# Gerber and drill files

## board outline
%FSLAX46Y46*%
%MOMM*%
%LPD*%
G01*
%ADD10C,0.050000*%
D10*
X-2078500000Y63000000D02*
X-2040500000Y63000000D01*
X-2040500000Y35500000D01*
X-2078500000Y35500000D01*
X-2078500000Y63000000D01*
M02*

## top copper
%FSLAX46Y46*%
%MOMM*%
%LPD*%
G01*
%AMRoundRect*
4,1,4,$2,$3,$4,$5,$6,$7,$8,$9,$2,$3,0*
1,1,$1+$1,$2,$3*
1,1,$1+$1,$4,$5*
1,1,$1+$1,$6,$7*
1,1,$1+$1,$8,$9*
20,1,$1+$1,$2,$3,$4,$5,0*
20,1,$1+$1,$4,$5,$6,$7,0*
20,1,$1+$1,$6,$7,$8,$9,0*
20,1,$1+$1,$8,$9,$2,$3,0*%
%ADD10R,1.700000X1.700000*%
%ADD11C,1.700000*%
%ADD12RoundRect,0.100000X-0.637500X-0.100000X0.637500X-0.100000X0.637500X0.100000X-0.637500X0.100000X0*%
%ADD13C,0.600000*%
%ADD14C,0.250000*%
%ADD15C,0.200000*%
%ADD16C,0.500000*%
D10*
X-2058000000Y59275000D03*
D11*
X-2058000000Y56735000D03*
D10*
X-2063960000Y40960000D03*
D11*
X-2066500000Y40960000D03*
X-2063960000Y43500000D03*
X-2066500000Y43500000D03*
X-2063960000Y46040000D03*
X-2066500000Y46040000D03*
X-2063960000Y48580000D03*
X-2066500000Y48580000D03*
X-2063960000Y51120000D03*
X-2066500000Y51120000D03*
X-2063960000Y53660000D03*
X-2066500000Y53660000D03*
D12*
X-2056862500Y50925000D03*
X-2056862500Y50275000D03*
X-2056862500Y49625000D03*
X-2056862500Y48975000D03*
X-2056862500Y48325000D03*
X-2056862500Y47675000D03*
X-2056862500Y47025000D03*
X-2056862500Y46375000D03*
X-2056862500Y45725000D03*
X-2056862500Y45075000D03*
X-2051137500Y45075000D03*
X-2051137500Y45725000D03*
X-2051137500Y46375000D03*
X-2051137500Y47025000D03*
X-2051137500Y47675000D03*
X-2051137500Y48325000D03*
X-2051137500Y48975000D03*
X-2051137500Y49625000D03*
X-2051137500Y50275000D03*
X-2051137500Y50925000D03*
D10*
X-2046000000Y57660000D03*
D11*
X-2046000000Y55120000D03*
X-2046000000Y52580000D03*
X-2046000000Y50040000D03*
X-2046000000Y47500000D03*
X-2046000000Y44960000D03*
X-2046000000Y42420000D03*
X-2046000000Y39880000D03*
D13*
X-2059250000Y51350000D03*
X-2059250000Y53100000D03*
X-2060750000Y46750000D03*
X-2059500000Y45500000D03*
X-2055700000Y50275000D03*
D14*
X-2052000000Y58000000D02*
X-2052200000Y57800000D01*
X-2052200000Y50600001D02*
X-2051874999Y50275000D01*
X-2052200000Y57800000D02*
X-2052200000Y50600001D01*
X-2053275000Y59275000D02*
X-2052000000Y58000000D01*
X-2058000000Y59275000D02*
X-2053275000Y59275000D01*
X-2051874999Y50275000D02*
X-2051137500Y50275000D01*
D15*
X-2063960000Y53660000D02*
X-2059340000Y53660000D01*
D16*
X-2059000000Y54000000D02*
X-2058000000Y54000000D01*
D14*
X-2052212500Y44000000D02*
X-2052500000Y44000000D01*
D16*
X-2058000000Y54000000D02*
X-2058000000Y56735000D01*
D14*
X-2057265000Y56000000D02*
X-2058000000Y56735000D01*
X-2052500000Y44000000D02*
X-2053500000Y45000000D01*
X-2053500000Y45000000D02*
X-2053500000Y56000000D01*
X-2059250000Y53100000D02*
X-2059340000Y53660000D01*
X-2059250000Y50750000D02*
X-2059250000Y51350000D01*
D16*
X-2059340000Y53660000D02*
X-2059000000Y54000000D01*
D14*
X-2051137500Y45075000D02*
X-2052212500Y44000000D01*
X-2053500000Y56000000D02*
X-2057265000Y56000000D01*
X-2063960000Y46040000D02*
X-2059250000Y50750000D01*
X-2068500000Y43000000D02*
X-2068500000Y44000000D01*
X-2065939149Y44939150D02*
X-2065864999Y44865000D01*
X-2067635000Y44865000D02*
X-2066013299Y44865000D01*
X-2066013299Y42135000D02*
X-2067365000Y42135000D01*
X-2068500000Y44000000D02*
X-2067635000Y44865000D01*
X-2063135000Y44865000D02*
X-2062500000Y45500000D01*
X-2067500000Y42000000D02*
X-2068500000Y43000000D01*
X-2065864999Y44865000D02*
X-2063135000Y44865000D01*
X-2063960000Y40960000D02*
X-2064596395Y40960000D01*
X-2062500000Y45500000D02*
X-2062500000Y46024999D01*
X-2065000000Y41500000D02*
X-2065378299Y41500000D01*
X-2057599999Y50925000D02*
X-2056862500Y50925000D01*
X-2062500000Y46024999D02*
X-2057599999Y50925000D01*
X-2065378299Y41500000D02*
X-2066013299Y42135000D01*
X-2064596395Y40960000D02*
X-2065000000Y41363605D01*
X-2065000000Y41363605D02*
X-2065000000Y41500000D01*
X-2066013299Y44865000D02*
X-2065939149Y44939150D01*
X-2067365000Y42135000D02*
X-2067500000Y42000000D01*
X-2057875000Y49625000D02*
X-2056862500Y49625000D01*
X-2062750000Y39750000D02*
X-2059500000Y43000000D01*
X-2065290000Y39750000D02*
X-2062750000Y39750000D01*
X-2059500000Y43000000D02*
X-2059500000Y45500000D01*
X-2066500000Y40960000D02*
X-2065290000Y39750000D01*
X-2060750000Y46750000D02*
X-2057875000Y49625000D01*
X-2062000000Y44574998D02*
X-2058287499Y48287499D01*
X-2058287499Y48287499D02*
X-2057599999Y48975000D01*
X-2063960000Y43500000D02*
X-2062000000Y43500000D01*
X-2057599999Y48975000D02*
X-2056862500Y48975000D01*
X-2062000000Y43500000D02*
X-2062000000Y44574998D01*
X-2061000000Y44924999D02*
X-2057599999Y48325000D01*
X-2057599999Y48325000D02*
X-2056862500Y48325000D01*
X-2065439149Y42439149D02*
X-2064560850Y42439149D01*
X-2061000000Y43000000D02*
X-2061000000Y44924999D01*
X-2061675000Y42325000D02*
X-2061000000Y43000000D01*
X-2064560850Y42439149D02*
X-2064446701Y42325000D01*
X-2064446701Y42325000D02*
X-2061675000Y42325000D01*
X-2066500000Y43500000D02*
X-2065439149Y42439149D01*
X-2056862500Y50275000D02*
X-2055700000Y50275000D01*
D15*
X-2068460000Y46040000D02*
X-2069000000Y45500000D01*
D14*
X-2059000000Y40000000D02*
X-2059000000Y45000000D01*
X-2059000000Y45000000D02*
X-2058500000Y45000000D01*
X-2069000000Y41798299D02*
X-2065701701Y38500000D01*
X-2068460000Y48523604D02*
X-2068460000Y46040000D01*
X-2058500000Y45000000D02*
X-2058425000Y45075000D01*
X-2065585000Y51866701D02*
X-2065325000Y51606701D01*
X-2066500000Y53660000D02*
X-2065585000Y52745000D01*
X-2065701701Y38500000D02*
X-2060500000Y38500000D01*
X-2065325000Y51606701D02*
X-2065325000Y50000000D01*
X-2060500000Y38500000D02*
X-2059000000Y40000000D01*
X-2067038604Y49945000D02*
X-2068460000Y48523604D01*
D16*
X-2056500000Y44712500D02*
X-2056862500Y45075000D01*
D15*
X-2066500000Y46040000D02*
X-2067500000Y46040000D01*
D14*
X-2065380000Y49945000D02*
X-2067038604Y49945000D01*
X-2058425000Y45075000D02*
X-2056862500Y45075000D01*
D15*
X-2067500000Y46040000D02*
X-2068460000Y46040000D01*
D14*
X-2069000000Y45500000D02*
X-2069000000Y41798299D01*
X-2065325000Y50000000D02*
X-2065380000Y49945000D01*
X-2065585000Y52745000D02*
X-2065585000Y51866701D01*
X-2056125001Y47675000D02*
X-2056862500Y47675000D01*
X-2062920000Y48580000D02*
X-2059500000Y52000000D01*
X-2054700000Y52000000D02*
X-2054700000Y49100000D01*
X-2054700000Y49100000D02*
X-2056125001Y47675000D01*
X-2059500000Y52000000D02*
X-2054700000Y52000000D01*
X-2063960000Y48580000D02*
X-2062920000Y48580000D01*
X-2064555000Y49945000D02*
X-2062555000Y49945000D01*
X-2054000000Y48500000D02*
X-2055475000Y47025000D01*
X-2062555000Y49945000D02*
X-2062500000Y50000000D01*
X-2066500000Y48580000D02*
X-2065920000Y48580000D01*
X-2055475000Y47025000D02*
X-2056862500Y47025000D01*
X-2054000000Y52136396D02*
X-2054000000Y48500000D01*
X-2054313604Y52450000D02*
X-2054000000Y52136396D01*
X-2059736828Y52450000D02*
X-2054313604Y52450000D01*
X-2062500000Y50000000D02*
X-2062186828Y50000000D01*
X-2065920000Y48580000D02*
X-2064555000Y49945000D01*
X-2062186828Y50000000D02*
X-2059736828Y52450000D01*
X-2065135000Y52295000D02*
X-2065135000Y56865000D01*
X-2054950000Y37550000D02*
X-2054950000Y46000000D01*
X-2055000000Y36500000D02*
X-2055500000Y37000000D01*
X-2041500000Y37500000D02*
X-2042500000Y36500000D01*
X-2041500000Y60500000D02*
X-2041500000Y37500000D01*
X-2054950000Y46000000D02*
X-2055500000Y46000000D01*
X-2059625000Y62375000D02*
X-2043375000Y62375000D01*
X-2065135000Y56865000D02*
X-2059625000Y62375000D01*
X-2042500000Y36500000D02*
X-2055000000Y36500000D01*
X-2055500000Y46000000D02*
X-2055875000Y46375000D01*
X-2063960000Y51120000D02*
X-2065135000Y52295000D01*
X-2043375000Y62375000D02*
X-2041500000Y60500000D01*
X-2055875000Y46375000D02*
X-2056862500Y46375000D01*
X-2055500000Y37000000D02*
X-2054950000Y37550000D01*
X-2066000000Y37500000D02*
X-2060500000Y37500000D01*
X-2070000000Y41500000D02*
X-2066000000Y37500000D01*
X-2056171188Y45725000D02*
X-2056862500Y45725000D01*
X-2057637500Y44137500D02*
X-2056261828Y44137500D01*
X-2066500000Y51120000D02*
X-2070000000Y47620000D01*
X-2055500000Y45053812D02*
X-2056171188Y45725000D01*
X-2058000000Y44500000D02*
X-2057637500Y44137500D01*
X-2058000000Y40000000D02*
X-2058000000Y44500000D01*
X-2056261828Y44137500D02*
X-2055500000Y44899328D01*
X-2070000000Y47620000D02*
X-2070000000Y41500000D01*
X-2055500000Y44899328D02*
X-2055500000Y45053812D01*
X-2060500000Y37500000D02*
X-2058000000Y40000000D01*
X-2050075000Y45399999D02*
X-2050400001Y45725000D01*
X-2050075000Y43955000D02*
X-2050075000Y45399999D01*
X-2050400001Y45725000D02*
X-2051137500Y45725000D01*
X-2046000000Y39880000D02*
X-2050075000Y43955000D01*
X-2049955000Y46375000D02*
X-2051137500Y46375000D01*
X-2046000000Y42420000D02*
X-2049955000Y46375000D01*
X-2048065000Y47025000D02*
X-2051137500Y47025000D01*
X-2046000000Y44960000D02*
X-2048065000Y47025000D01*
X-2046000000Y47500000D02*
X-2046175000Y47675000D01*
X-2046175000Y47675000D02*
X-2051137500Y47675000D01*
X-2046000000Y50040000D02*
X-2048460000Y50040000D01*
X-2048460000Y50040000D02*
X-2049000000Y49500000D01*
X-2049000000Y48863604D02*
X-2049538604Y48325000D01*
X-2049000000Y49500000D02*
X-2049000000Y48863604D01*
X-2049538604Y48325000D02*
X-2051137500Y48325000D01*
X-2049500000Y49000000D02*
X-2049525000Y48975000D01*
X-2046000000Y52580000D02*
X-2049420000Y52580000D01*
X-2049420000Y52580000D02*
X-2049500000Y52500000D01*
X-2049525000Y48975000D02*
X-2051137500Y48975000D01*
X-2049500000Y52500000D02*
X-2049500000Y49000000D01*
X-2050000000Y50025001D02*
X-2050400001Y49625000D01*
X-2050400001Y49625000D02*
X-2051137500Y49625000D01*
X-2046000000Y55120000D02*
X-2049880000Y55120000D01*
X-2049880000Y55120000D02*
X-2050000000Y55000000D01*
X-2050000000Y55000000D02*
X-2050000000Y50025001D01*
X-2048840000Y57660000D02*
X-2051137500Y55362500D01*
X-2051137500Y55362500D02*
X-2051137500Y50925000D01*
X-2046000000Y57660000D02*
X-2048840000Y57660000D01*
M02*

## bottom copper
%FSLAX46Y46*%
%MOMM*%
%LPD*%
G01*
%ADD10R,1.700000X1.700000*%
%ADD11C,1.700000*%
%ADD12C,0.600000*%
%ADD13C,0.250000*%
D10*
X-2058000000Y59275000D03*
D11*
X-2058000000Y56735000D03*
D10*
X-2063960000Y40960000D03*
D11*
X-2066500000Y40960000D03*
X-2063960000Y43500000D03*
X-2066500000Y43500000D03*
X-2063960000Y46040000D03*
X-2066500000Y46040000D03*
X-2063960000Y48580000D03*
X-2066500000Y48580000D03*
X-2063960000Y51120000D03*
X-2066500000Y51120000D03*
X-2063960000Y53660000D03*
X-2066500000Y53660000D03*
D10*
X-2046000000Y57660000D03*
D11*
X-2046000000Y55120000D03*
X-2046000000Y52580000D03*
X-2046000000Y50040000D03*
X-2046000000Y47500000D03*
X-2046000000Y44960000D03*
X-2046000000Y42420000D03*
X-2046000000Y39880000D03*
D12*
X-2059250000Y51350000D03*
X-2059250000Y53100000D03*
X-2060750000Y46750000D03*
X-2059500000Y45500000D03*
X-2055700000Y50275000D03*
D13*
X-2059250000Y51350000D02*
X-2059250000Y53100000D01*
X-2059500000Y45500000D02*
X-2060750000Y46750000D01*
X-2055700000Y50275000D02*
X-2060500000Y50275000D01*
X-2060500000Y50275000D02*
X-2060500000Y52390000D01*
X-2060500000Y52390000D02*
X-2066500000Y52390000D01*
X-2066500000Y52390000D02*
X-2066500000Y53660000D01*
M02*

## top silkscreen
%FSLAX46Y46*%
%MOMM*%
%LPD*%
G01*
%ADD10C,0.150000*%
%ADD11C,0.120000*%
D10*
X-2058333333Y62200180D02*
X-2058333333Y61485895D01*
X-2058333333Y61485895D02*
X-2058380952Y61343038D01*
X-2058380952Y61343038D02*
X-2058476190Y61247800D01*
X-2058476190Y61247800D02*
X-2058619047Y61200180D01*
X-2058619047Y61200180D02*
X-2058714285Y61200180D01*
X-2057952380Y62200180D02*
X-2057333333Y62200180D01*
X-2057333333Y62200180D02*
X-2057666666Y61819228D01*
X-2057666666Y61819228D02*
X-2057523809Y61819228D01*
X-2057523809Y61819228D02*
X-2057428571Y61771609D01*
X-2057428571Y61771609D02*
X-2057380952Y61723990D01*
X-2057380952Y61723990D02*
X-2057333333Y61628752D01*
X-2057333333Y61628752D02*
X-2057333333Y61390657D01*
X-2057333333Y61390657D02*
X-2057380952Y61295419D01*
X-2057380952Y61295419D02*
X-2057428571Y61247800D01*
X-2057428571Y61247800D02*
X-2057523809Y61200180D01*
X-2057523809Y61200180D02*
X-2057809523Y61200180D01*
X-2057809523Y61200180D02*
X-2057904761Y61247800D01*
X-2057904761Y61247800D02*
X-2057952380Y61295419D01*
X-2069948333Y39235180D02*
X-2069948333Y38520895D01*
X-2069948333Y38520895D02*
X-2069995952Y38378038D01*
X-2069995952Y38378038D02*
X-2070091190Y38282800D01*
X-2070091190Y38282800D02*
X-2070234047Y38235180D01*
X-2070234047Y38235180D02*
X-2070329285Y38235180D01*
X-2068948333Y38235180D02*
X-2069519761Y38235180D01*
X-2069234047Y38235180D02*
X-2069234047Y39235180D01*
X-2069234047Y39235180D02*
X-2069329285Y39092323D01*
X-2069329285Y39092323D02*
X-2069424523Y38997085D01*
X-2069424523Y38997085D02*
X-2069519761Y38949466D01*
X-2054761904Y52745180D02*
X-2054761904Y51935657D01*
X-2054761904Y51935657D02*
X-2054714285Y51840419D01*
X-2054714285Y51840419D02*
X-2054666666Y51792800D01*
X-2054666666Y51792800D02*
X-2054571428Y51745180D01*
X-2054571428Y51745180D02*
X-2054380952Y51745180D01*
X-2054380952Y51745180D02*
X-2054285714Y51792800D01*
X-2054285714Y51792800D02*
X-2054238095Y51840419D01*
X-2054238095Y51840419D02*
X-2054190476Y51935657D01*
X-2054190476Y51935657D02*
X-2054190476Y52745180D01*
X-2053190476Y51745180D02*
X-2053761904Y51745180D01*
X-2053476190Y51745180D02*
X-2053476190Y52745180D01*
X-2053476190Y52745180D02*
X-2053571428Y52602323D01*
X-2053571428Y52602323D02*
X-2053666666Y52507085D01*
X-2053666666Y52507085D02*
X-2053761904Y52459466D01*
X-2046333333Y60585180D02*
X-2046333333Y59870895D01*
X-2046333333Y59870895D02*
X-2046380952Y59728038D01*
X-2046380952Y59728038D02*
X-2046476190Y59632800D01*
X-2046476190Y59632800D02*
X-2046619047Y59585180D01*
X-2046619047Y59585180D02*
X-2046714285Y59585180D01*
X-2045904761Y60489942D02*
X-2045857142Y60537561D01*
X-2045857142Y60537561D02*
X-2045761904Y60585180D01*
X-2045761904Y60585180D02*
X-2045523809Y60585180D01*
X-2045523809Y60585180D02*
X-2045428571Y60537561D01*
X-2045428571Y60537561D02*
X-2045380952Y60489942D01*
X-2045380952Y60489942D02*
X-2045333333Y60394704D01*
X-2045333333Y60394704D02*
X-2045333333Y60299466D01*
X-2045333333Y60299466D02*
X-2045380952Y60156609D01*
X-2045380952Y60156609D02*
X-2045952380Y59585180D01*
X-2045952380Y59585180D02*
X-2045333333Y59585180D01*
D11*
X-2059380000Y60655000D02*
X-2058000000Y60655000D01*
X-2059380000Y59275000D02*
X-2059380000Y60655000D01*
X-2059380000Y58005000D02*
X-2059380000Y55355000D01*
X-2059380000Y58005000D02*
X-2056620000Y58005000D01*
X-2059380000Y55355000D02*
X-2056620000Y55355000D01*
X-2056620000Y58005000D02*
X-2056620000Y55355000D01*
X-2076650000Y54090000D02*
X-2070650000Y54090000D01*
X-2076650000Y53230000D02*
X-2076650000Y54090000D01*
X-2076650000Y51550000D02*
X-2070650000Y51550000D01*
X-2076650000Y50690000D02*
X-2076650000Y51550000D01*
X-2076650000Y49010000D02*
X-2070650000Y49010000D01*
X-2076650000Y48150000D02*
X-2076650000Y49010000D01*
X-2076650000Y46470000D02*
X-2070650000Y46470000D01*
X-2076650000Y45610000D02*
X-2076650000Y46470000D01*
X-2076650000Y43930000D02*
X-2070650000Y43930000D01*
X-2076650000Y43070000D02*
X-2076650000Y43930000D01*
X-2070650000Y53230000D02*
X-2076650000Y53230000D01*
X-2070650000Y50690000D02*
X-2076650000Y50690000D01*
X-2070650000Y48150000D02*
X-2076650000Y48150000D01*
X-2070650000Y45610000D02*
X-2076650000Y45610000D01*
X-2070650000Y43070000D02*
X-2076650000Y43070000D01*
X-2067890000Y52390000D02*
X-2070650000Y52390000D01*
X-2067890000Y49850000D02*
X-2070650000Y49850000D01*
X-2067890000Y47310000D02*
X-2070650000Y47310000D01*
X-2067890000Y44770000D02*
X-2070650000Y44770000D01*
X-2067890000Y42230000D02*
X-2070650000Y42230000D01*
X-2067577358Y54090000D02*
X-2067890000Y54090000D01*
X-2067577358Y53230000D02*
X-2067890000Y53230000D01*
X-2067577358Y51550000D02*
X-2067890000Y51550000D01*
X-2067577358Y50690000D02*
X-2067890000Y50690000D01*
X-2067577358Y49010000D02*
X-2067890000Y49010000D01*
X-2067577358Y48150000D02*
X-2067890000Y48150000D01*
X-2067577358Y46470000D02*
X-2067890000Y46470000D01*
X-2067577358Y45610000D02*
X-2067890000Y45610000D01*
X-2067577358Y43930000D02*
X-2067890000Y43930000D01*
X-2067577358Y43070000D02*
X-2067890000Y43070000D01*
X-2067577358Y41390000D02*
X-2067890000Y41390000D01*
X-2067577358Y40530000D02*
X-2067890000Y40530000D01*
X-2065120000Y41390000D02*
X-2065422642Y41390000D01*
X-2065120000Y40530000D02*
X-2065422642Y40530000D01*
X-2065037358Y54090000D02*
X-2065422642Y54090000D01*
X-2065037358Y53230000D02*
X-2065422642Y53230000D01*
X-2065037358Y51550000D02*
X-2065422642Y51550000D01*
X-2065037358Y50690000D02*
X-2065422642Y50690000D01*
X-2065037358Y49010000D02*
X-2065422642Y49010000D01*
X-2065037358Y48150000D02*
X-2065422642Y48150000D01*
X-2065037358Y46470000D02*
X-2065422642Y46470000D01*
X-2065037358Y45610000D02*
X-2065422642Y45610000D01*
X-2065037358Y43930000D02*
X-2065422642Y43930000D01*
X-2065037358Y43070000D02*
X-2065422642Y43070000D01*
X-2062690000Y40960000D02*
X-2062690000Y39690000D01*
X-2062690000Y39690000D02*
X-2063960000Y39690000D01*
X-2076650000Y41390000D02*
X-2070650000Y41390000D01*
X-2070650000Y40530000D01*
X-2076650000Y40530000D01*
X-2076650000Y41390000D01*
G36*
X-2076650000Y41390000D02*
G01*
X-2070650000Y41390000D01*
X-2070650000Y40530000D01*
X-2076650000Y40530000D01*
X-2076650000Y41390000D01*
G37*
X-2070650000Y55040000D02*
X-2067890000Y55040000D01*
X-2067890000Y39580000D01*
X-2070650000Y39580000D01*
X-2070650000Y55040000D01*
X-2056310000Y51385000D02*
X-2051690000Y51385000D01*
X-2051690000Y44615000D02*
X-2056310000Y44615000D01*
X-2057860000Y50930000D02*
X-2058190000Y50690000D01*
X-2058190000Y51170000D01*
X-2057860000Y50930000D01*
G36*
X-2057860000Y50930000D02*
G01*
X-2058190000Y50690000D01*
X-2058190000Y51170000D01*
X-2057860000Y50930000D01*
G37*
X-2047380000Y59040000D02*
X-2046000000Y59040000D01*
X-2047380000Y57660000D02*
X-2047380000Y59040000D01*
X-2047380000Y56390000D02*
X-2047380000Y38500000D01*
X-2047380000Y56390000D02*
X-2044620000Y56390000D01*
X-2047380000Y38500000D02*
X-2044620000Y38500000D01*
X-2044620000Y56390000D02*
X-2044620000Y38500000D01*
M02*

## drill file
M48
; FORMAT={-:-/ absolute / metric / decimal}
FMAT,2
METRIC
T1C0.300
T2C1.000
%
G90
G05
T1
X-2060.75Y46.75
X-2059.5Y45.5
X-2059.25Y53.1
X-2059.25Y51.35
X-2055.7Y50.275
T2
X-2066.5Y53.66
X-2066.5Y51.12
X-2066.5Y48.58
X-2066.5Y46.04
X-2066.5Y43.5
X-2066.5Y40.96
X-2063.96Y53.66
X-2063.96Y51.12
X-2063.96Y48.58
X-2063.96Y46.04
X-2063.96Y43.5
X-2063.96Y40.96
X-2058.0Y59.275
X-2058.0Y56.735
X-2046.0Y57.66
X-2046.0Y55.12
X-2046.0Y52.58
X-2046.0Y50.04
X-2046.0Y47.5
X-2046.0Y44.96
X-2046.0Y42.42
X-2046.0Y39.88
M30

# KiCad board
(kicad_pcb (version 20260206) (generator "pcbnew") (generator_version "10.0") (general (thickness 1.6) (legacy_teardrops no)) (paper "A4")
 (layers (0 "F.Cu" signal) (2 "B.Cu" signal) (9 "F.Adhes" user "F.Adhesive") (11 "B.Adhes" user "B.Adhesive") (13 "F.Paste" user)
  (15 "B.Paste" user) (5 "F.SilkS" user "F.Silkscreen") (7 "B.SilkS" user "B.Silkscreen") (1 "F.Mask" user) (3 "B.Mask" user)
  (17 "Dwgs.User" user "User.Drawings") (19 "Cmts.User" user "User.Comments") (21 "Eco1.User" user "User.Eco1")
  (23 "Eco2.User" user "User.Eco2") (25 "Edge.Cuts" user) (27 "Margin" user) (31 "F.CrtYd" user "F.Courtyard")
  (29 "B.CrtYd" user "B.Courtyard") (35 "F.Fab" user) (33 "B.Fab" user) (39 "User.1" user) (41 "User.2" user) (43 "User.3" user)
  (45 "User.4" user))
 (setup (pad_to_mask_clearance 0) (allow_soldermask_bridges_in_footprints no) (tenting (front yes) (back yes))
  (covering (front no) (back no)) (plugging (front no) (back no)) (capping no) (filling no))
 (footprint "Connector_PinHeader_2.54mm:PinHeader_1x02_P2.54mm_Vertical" (layer "F.Cu") (at -2058 -59.275)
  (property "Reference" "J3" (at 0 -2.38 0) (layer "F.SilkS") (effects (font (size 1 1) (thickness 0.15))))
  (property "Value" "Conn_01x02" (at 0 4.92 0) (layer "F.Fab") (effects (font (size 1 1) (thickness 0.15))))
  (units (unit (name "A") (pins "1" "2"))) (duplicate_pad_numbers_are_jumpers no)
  (fp_line (start -1.38 -1.38) (end 0 -1.38) (stroke (width 0.12) (type solid)) (layer "F.SilkS"))
  (fp_line (start -1.38 0) (end -1.38 -1.38) (stroke (width 0.12) (type solid)) (layer "F.SilkS"))
  (fp_line (start -1.38 1.27) (end -1.38 3.92) (stroke (width 0.12) (type solid)) (layer "F.SilkS"))
  (fp_line (start -1.38 1.27) (end 1.38 1.27) (stroke (width 0.12) (type solid)) (layer "F.SilkS"))
  (fp_line (start -1.38 3.92) (end 1.38 3.92) (stroke (width 0.12) (type solid)) (layer "F.SilkS"))
  (fp_line (start 1.38 1.27) (end 1.38 3.92) (stroke (width 0.12) (type solid)) (layer "F.SilkS"))
  (pad "1" thru_hole rect (at 0 0) (size 1.7 1.7) (drill 1) (layers "*.Cu" "*.Mask") (remove_unused_layers no) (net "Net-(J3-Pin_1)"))
  (pad "2" thru_hole circle (at 0 2.54) (size 1.7 1.7) (drill 1) (layers "*.Cu" "*.Mask") (remove_unused_layers no) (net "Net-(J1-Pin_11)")))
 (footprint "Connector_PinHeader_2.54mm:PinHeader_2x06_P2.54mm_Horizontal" (layer "F.Cu") (at -2063.96 -40.96 180)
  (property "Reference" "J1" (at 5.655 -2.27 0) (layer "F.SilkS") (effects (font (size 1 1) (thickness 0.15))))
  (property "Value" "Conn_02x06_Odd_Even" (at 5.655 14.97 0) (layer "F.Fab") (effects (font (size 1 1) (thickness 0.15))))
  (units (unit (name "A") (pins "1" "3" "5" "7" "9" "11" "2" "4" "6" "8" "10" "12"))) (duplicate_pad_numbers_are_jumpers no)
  (fp_line (start 12.69 13.13) (end 6.69 13.13) (stroke (width 0.12) (type solid)) (layer "F.SilkS"))
  (fp_line (start 12.69 12.27) (end 12.69 13.13) (stroke (width 0.12) (type solid)) (layer "F.SilkS"))
  (fp_line (start 12.69 10.59) (end 6.69 10.59) (stroke (width 0.12) (type solid)) (layer "F.SilkS"))
  (fp_line (start 12.69 9.73) (end 12.69 10.59) (stroke (width 0.12) (type solid)) (layer "F.SilkS"))
  (fp_line (start 12.69 8.05) (end 6.69 8.05) (stroke (width 0.12) (type solid)) (layer "F.SilkS"))
  (fp_line (start 12.69 7.19) (end 12.69 8.05) (stroke (width 0.12) (type solid)) (layer "F.SilkS"))
  (fp_line (start 12.69 5.51) (end 6.69 5.51) (stroke (width 0.12) (type solid)) (layer "F.SilkS"))
  (fp_line (start 12.69 4.65) (end 12.69 5.51) (stroke (width 0.12) (type solid)) (layer "F.SilkS"))
  (fp_line (start 12.69 2.97) (end 6.69 2.97) (stroke (width 0.12) (type solid)) (layer "F.SilkS"))
  (fp_line (start 12.69 2.11) (end 12.69 2.97) (stroke (width 0.12) (type solid)) (layer "F.SilkS"))
  (fp_line (start 6.69 12.27) (end 12.69 12.27) (stroke (width 0.12) (type solid)) (layer "F.SilkS"))
  (fp_line (start 6.69 9.73) (end 12.69 9.73) (stroke (width 0.12) (type solid)) (layer "F.SilkS"))
  (fp_line (start 6.69 7.19) (end 12.69 7.19) (stroke (width 0.12) (type solid)) (layer "F.SilkS"))
  (fp_line (start 6.69 4.65) (end 12.69 4.65) (stroke (width 0.12) (type solid)) (layer "F.SilkS"))
  (fp_line (start 6.69 2.11) (end 12.69 2.11) (stroke (width 0.12) (type solid)) (layer "F.SilkS"))
  (fp_line (start 3.93 11.43) (end 6.69 11.43) (stroke (width 0.12) (type solid)) (layer "F.SilkS"))
  (fp_line (start 3.93 8.89) (end 6.69 8.89) (stroke (width 0.12) (type solid)) (layer "F.SilkS"))
  (fp_line (start 3.93 6.35) (end 6.69 6.35) (stroke (width 0.12) (type solid)) (layer "F.SilkS"))
  (fp_line (start 3.93 3.81) (end 6.69 3.81) (stroke (width 0.12) (type solid)) (layer "F.SilkS"))
  (fp_line (start 3.93 1.27) (end 6.69 1.27) (stroke (width 0.12) (type solid)) (layer "F.SilkS"))
  (fp_line (start 3.617358 13.13) (end 3.93 13.13) (stroke (width 0.12) (type solid)) (layer "F.SilkS"))
  (fp_line (start 3.617358 12.27) (end 3.93 12.27) (stroke (width 0.12) (type solid)) (layer "F.SilkS"))
  (fp_line (start 3.617358 10.59) (end 3.93 10.59) (stroke (width 0.12) (type solid)) (layer "F.SilkS"))
  (fp_line (start 3.617358 9.73) (end 3.93 9.73) (stroke (width 0.12) (type solid)) (layer "F.SilkS"))
  (fp_line (start 3.617358 8.05) (end 3.93 8.05) (stroke (width 0.12) (type solid)) (layer "F.SilkS"))
  (fp_line (start 3.617358 7.19) (end 3.93 7.19) (stroke (width 0.12) (type solid)) (layer "F.SilkS"))
  (fp_line (start 3.617358 5.51) (end 3.93 5.51) (stroke (width 0.12) (type solid)) (layer "F.SilkS"))
  (fp_line (start 3.617358 4.65) (end 3.93 4.65) (stroke (width 0.12) (type solid)) (layer "F.SilkS"))
  (fp_line (start 3.617358 2.97) (end 3.93 2.97) (stroke (width 0.12) (type solid)) (layer "F.SilkS"))
  (fp_line (start 3.617358 2.11) (end 3.93 2.11) (stroke (width 0.12) (type solid)) (layer "F.SilkS"))
  (fp_line (start 3.617358 0.43) (end 3.93 0.43) (stroke (width 0.12) (type solid)) (layer "F.SilkS"))
  (fp_line (start 3.617358 -0.43) (end 3.93 -0.43) (stroke (width 0.12) (type solid)) (layer "F.SilkS"))
  (fp_line (start 1.16 0.43) (end 1.462642 0.43) (stroke (width 0.12) (type solid)) (layer "F.SilkS"))
  (fp_line (start 1.16 -0.43) (end 1.462642 -0.43) (stroke (width 0.12) (type solid)) (layer "F.SilkS"))
  (fp_line (start 1.077358 13.13) (end 1.462642 13.13) (stroke (width 0.12) (type solid)) (layer "F.SilkS"))
  (fp_line (start 1.077358 12.27) (end 1.462642 12.27) (stroke (width 0.12) (type solid)) (layer "F.SilkS"))
  (fp_line (start 1.077358 10.59) (end 1.462642 10.59) (stroke (width 0.12) (type solid)) (layer "F.SilkS"))
  (fp_line (start 1.077358 9.73) (end 1.462642 9.73) (stroke (width 0.12) (type solid)) (layer "F.SilkS"))
  (fp_line (start 1.077358 8.05) (end 1.462642 8.05) (stroke (width 0.12) (type solid)) (layer "F.SilkS"))
  (fp_line (start 1.077358 7.19) (end 1.462642 7.19) (stroke (width 0.12) (type solid)) (layer "F.SilkS"))
  (fp_line (start 1.077358 5.51) (end 1.462642 5.51) (stroke (width 0.12) (type solid)) (layer "F.SilkS"))
  (fp_line (start 1.077358 4.65) (end 1.462642 4.65) (stroke (width 0.12) (type solid)) (layer "F.SilkS"))
  (fp_line (start 1.077358 2.97) (end 1.462642 2.97) (stroke (width 0.12) (type solid)) (layer "F.SilkS"))
  (fp_line (start 1.077358 2.11) (end 1.462642 2.11) (stroke (width 0.12) (type solid)) (layer "F.SilkS"))
  (fp_line (start -1.27 0) (end -1.27 -1.27) (stroke (width 0.12) (type solid)) (layer "F.SilkS"))
  (fp_line (start -1.27 -1.27) (end 0 -1.27) (stroke (width 0.12) (type solid)) (layer "F.SilkS"))
  (fp_rect (start 6.69 -0.43) (end 12.69 0.43) (stroke (width 0.12) (type solid)) (fill yes) (layer "F.SilkS"))
  (fp_rect (start 3.93 -1.38) (end 6.69 14.08) (stroke (width 0.12) (type solid)) (fill no) (layer "F.SilkS"))
  (pad "1" thru_hole rect (at 0 0 180) (size 1.7 1.7) (drill 1) (layers "*.Cu" "*.Mask") (remove_unused_layers no) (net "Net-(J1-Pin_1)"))
  (pad "2" thru_hole circle (at 2.54 0 180) (size 1.7 1.7) (drill 1) (layers "*.Cu" "*.Mask") (remove_unused_layers no)
   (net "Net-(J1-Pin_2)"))
  (pad "3" thru_hole circle (at 0 2.54 180) (size 1.7 1.7) (drill 1) (layers "*.Cu" "*.Mask") (remove_unused_layers no)
   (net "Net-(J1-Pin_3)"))
  (pad "4" thru_hole circle (at 2.54 2.54 180) (size 1.7 1.7) (drill 1) (layers "*.Cu" "*.Mask") (remove_unused_layers no)
   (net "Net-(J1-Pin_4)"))
  (pad "5" thru_hole circle (at 0 5.08 180) (size 1.7 1.7) (drill 1) (layers "*.Cu" "*.Mask") (remove_unused_layers no)
   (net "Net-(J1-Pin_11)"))
  (pad "6" thru_hole circle (at 2.54 5.08 180) (size 1.7 1.7) (drill 1) (layers "*.Cu" "*.Mask") (remove_unused_layers no)
   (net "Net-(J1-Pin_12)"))
  (pad "7" thru_hole circle (at 0 7.62 180) (size 1.7 1.7) (drill 1) (layers "*.Cu" "*.Mask") (remove_unused_layers no)
   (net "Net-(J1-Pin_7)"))
  (pad "8" thru_hole circle (at 2.54 7.62 180) (size 1.7 1.7) (drill 1) (layers "*.Cu" "*.Mask") (remove_unused_layers no)
   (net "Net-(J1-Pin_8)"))
  (pad "9" thru_hole circle (at 0 10.16 180) (size 1.7 1.7) (drill 1) (layers "*.Cu" "*.Mask") (remove_unused_layers no)
   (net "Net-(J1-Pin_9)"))
  (pad "10" thru_hole circle (at 2.54 10.16 180) (size 1.7 1.7) (drill 1) (layers "*.Cu" "*.Mask") (remove_unused_layers no)
   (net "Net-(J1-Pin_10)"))
  (pad "11" thru_hole circle (at 0 12.7 180) (size 1.7 1.7) (drill 1) (layers "*.Cu" "*.Mask") (remove_unused_layers no)
   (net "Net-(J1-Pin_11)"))
  (pad "12" thru_hole circle (at 2.54 12.7 180) (size 1.7 1.7) (drill 1) (layers "*.Cu" "*.Mask") (remove_unused_layers no)
   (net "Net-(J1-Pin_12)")))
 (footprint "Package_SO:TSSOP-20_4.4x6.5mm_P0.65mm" (layer "F.Cu") (at -2054 -48)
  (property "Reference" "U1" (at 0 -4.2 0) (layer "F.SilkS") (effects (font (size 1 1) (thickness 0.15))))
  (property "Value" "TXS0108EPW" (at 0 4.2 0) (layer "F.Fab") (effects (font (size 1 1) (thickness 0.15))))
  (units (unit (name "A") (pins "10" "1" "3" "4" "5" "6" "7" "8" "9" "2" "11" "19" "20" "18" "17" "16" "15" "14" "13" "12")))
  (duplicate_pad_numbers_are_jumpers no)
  (fp_line (start -2.31 -3.385) (end 2.31 -3.385) (stroke (width 0.12) (type solid)) (layer "F.SilkS"))
  (fp_line (start 2.31 3.385) (end -2.31 3.385) (stroke (width 0.12) (type solid)) (layer "F.SilkS"))
  (fp_poly (pts (xy -3.86 -2.93) (xy -4.19 -2.69) (xy -4.19 -3.17)) (stroke (width 0.12) (type solid)) (fill yes) (layer "F.SilkS"))
  (pad "1" smd roundrect (at -2.8625 -2.925) (size 1.475 0.4) (layers "F.Cu" "F.Mask" "F.Paste") (roundrect_rratio 0.25)
   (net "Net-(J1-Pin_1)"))
  (pad "2" smd roundrect (at -2.8625 -2.275) (size 1.475 0.4) (layers "F.Cu" "F.Mask" "F.Paste") (roundrect_rratio 0.25)
   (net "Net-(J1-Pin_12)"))
  (pad "3" smd roundrect (at -2.8625 -1.625) (size 1.475 0.4) (layers "F.Cu" "F.Mask" "F.Paste") (roundrect_rratio 0.25)
   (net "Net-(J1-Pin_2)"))
  (pad "4" smd roundrect (at -2.8625 -0.975) (size 1.475 0.4) (layers "F.Cu" "F.Mask" "F.Paste") (roundrect_rratio 0.25)
   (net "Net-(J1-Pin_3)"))
  (pad "5" smd roundrect (at -2.8625 -0.325) (size 1.475 0.4) (layers "F.Cu" "F.Mask" "F.Paste") (roundrect_rratio 0.25)
   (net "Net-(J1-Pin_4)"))
  (pad "6" smd roundrect (at -2.8625 0.325) (size 1.475 0.4) (layers "F.Cu" "F.Mask" "F.Paste") (roundrect_rratio 0.25)
   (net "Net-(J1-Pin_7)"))
  (pad "7" smd roundrect (at -2.8625 0.975) (size 1.475 0.4) (layers "F.Cu" "F.Mask" "F.Paste") (roundrect_rratio 0.25)
   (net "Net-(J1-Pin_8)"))
  (pad "8" smd roundrect (at -2.8625 1.625) (size 1.475 0.4) (layers "F.Cu" "F.Mask" "F.Paste") (roundrect_rratio 0.25)
   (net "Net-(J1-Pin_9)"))
  (pad "9" smd roundrect (at -2.8625 2.275) (size 1.475 0.4) (layers "F.Cu" "F.Mask" "F.Paste") (roundrect_rratio 0.25)
   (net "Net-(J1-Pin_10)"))
  (pad "10" smd roundrect (at -2.8625 2.925) (size 1.475 0.4) (layers "F.Cu" "F.Mask" "F.Paste") (roundrect_rratio 0.25)
   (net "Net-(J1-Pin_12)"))
  (pad "11" smd roundrect (at 2.8625 2.925) (size 1.475 0.4) (layers "F.Cu" "F.Mask" "F.Paste") (roundrect_rratio 0.25)
   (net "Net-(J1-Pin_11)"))
  (pad "12" smd roundrect (at 2.8625 2.275) (size 1.475 0.4) (layers "F.Cu" "F.Mask" "F.Paste") (roundrect_rratio 0.25)
   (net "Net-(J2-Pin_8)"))
  (pad "13" smd roundrect (at 2.8625 1.625) (size 1.475 0.4) (layers "F.Cu" "F.Mask" "F.Paste") (roundrect_rratio 0.25)
   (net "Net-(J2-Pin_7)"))
  (pad "14" smd roundrect (at 2.8625 0.975) (size 1.475 0.4) (layers "F.Cu" "F.Mask" "F.Paste") (roundrect_rratio 0.25)
   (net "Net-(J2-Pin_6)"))
  (pad "15" smd roundrect (at 2.8625 0.325) (size 1.475 0.4) (layers "F.Cu" "F.Mask" "F.Paste") (roundrect_rratio 0.25)
   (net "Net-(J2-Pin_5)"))
  (pad "16" smd roundrect (at 2.8625 -0.325) (size 1.475 0.4) (layers "F.Cu" "F.Mask" "F.Paste") (roundrect_rratio 0.25)
   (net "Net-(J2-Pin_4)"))
  (pad "17" smd roundrect (at 2.8625 -0.975) (size 1.475 0.4) (layers "F.Cu" "F.Mask" "F.Paste") (roundrect_rratio 0.25)
   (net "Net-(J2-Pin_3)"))
  (pad "18" smd roundrect (at 2.8625 -1.625) (size 1.475 0.4) (layers "F.Cu" "F.Mask" "F.Paste") (roundrect_rratio 0.25)
   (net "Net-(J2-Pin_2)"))
  (pad "19" smd roundrect (at 2.8625 -2.275) (size 1.475 0.4) (layers "F.Cu" "F.Mask" "F.Paste") (roundrect_rratio 0.25)
   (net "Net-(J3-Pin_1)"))
  (pad "20" smd roundrect (at 2.8625 -2.925) (size 1.475 0.4) (layers "F.Cu" "F.Mask" "F.Paste") (roundrect_rratio 0.25)
   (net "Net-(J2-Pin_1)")))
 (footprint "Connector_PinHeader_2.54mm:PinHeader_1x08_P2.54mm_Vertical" (layer "F.Cu") (at -2046 -57.66)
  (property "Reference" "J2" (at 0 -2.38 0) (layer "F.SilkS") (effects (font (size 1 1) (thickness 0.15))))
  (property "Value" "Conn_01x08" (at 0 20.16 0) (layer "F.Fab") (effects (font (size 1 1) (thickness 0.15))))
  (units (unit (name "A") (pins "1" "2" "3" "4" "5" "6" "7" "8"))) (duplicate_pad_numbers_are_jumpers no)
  (fp_line (start -1.38 -1.38) (end 0 -1.38) (stroke (width 0.12) (type solid)) (layer "F.SilkS"))
  (fp_line (start -1.38 0) (end -1.38 -1.38) (stroke (width 0.12) (type solid)) (layer "F.SilkS"))
  (fp_line (start -1.38 1.27) (end -1.38 19.16) (stroke (width 0.12) (type solid)) (layer "F.SilkS"))
  (fp_line (start -1.38 1.27) (end 1.38 1.27) (stroke (width 0.12) (type solid)) (layer "F.SilkS"))
  (fp_line (start -1.38 19.16) (end 1.38 19.16) (stroke (width 0.12) (type solid)) (layer "F.SilkS"))
  (fp_line (start 1.38 1.27) (end 1.38 19.16) (stroke (width 0.12) (type solid)) (layer "F.SilkS"))
  (pad "1" thru_hole rect (at 0 0) (size 1.7 1.7) (drill 1) (layers "*.Cu" "*.Mask") (remove_unused_layers no) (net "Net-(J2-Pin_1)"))
  (pad "2" thru_hole circle (at 0 2.54) (size 1.7 1.7) (drill 1) (layers "*.Cu" "*.Mask") (remove_unused_layers no) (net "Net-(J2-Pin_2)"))
  (pad "3" thru_hole circle (at 0 5.08) (size 1.7 1.7) (drill 1) (layers "*.Cu" "*.Mask") (remove_unused_layers no) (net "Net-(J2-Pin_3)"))
  (pad "4" thru_hole circle (at 0 7.62) (size 1.7 1.7) (drill 1) (layers "*.Cu" "*.Mask") (remove_unused_layers no) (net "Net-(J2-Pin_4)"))
  (pad "5" thru_hole circle (at 0 10.16) (size 1.7 1.7) (drill 1) (layers "*.Cu" "*.Mask") (remove_unused_layers no) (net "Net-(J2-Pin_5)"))
  (pad "6" thru_hole circle (at 0 12.7) (size 1.7 1.7) (drill 1) (layers "*.Cu" "*.Mask") (remove_unused_layers no) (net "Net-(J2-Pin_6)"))
  (pad "7" thru_hole circle (at 0 15.24) (size 1.7 1.7) (drill 1) (layers "*.Cu" "*.Mask") (remove_unused_layers no) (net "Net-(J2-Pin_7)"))
  (pad "8" thru_hole circle (at 0 17.78) (size 1.7 1.7) (drill 1) (layers "*.Cu" "*.Mask") (remove_unused_layers no) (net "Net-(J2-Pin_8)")))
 (gr_rect (start -2078.5 -63) (end -2040.5 -35.5) (stroke (width 0.05) (type default)) (fill no) (layer "Edge.Cuts"))
 (segment (start -2052 -58) (end -2052.2 -57.8) (width 0.25) (layer "F.Cu") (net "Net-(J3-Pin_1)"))
 (segment (start -2052.2 -50.600001) (end -2051.874999 -50.275) (width 0.25) (layer "F.Cu") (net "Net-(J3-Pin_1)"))
 (segment (start -2052.2 -57.8) (end -2052.2 -50.600001) (width 0.25) (layer "F.Cu") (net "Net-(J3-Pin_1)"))
 (segment (start -2053.275 -59.275) (end -2052 -58) (width 0.25) (layer "F.Cu") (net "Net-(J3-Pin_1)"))
 (segment (start -2058 -59.275) (end -2053.275 -59.275) (width 0.25) (layer "F.Cu") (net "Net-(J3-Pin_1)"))
 (segment (start -2051.874999 -50.275) (end -2051.1375 -50.275) (width 0.25) (layer "F.Cu") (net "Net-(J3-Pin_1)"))
 (segment (start -2063.96 -53.66) (end -2059.34 -53.66) (width 0.2) (layer "F.Cu") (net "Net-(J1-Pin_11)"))
 (segment (start -2059 -54) (end -2058 -54) (width 0.5) (layer "F.Cu") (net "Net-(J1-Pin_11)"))
 (segment (start -2052.2125 -44) (end -2052.5 -44) (width 0.25) (layer "F.Cu") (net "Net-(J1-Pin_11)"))
 (segment (start -2058 -54) (end -2058 -56.735) (width 0.5) (layer "F.Cu") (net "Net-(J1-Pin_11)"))
 (segment (start -2057.265 -56) (end -2058 -56.735) (width 0.25) (layer "F.Cu") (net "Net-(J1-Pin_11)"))
 (segment (start -2052.5 -44) (end -2053.5 -45) (width 0.25) (layer "F.Cu") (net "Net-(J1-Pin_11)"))
 (segment (start -2053.5 -45) (end -2053.5 -56) (width 0.25) (layer "F.Cu") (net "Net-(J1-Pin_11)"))
 (segment (start -2059.25 -53.1) (end -2059.34 -53.66) (width 0.25) (layer "F.Cu") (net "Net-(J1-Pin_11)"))
 (segment (start -2059.25 -50.75) (end -2059.25 -51.35) (width 0.25) (layer "F.Cu") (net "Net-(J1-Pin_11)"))
 (segment (start -2059.34 -53.66) (end -2059 -54) (width 0.5) (layer "F.Cu") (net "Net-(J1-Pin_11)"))
 (segment (start -2051.1375 -45.075) (end -2052.2125 -44) (width 0.25) (layer "F.Cu") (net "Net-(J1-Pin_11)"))
 (segment (start -2053.5 -56) (end -2057.265 -56) (width 0.25) (layer "F.Cu") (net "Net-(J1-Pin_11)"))
 (segment (start -2063.96 -46.04) (end -2059.25 -50.75) (width 0.25) (layer "F.Cu") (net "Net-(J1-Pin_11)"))
 (via (at -2059.25 -51.35) (size 0.6) (drill 0.3) (layers "F.Cu" "B.Cu") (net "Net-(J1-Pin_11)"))
 (via (at -2059.25 -53.1) (size 0.6) (drill 0.3) (layers "F.Cu" "B.Cu") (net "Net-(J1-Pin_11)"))
 (segment (start -2059.25 -51.35) (end -2059.25 -53.1) (width 0.25) (layer "B.Cu") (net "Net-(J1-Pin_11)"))
 (segment (start -2068.5 -43) (end -2068.5 -44) (width 0.25) (layer "F.Cu") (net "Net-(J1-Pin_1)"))
 (segment (start -2065.939149 -44.93915) (end -2065.864999 -44.865) (width 0.25) (layer "F.Cu") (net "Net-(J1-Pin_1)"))
 (segment (start -2067.635 -44.865) (end -2066.013299 -44.865) (width 0.25) (layer "F.Cu") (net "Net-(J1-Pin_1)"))
 (segment (start -2066.013299 -42.135) (end -2067.365 -42.135) (width 0.25) (layer "F.Cu") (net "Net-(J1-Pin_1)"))
 (segment (start -2068.5 -44) (end -2067.635 -44.865) (width 0.25) (layer "F.Cu") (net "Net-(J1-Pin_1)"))
 (segment (start -2063.135 -44.865) (end -2062.5 -45.5) (width 0.25) (layer "F.Cu") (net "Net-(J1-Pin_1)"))
 (segment (start -2067.5 -42) (end -2068.5 -43) (width 0.25) (layer "F.Cu") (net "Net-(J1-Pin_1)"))
 (segment (start -2065.864999 -44.865) (end -2063.135 -44.865) (width 0.25) (layer "F.Cu") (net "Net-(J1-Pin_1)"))
 (segment (start -2063.96 -40.96) (end -2064.596395 -40.96) (width 0.25) (layer "F.Cu") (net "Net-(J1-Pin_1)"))
 (segment (start -2062.5 -45.5) (end -2062.5 -46.024999) (width 0.25) (layer "F.Cu") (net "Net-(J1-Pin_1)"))
 (segment (start -2065 -41.5) (end -2065.378299 -41.5) (width 0.25) (layer "F.Cu") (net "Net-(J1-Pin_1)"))
 (segment (start -2057.599999 -50.925) (end -2056.8625 -50.925) (width 0.25) (layer "F.Cu") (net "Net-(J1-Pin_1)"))
 (segment (start -2062.5 -46.024999) (end -2057.599999 -50.925) (width 0.25) (layer "F.Cu") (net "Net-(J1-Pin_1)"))
 (segment (start -2065.378299 -41.5) (end -2066.013299 -42.135) (width 0.25) (layer "F.Cu") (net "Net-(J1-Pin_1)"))
 (segment (start -2064.596395 -40.96) (end -2065 -41.363605) (width 0.25) (layer "F.Cu") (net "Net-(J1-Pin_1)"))
 (segment (start -2065 -41.363605) (end -2065 -41.5) (width 0.25) (layer "F.Cu") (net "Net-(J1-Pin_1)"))
 (segment (start -2066.013299 -44.865) (end -2065.939149 -44.93915) (width 0.25) (layer "F.Cu") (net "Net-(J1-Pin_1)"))
 (segment (start -2067.365 -42.135) (end -2067.5 -42) (width 0.25) (layer "F.Cu") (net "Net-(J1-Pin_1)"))
 (segment (start -2057.875 -49.625) (end -2056.8625 -49.625) (width 0.25) (layer "F.Cu") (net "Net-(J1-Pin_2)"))
 (segment (start -2062.75 -39.75) (end -2059.5 -43) (width 0.25) (layer "F.Cu") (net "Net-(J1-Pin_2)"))
 (segment (start -2065.29 -39.75) (end -2062.75 -39.75) (width 0.25) (layer "F.Cu") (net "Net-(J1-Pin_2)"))
 (segment (start -2059.5 -43) (end -2059.5 -45.5) (width 0.25) (layer "F.Cu") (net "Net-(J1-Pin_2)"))
 (segment (start -2066.5 -40.96) (end -2065.29 -39.75) (width 0.25) (layer "F.Cu") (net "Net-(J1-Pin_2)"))
 (segment (start -2060.75 -46.75) (end -2057.875 -49.625) (width 0.25) (layer "F.Cu") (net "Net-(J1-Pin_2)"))
 (via (at -2060.75 -46.75) (size 0.6) (drill 0.3) (layers "F.Cu" "B.Cu") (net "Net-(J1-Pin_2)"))
 (via (at -2059.5 -45.5) (size 0.6) (drill 0.3) (layers "F.Cu" "B.Cu") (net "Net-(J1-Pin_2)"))
 (segment (start -2059.5 -45.5) (end -2060.75 -46.75) (width 0.25) (layer "B.Cu") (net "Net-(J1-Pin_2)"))
 (segment (start -2062 -44.574998) (end -2058.287499 -48.287499) (width 0.25) (layer "F.Cu") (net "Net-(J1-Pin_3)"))
 (segment (start -2058.287499 -48.287499) (end -2057.599999 -48.975) (width 0.25) (layer "F.Cu") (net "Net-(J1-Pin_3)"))
 (segment (start -2063.96 -43.5) (end -2062 -43.5) (width 0.25) (layer "F.Cu") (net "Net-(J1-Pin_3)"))
 (segment (start -2057.599999 -48.975) (end -2056.8625 -48.975) (width 0.25) (layer "F.Cu") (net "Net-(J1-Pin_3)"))
 (segment (start -2062 -43.5) (end -2062 -44.574998) (width 0.25) (layer "F.Cu") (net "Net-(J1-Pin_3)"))
 (segment (start -2061 -44.924999) (end -2057.599999 -48.325) (width 0.25) (layer "F.Cu") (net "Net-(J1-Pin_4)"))
 (segment (start -2057.599999 -48.325) (end -2056.8625 -48.325) (width 0.25) (layer "F.Cu") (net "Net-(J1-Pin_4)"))
 (segment (start -2065.439149 -42.439149) (end -2064.56085 -42.439149) (width 0.25) (layer "F.Cu") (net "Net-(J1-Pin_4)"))
 (segment (start -2061 -43) (end -2061 -44.924999) (width 0.25) (layer "F.Cu") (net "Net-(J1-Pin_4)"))
 (segment (start -2061.675 -42.325) (end -2061 -43) (width 0.25) (layer "F.Cu") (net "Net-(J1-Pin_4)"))
 (segment (start -2064.56085 -42.439149) (end -2064.446701 -42.325) (width 0.25) (layer "F.Cu") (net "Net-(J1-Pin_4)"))
 (segment (start -2064.446701 -42.325) (end -2061.675 -42.325) (width 0.25) (layer "F.Cu") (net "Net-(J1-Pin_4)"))
 (segment (start -2066.5 -43.5) (end -2065.439149 -42.439149) (width 0.25) (layer "F.Cu") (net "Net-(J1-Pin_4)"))
 (segment (start -2056.8625 -50.275) (end -2055.7 -50.275) (width 0.25) (layer "F.Cu") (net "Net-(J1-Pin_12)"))
 (via (at -2055.7 -50.275) (size 0.6) (drill 0.3) (layers "F.Cu" "B.Cu") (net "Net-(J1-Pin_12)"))
 (segment (start -2055.7 -50.275) (end -2060.5 -50.275) (width 0.25) (layer "B.Cu") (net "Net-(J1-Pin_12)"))
 (segment (start -2060.5 -50.275) (end -2060.5 -52.39) (width 0.25) (layer "B.Cu") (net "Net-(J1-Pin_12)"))
 (segment (start -2060.5 -52.39) (end -2066.5 -52.39) (width 0.25) (layer "B.Cu") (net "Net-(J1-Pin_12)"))
 (segment (start -2066.5 -52.39) (end -2066.5 -53.66) (width 0.25) (layer "B.Cu") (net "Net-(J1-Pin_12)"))
 (segment (start -2068.46 -46.04) (end -2069 -45.5) (width 0.2) (layer "F.Cu") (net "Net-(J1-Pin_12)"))
 (segment (start -2059 -40) (end -2059 -45) (width 0.25) (layer "F.Cu") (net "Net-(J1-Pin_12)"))
 (segment (start -2059 -45) (end -2058.5 -45) (width 0.25) (layer "F.Cu") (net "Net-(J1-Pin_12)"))
 (segment (start -2069 -41.798299) (end -2065.701701 -38.5) (width 0.25) (layer "F.Cu") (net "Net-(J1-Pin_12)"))
 (segment (start -2068.46 -48.523604) (end -2068.46 -46.04) (width 0.25) (layer "F.Cu") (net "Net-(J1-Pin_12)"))
 (segment (start -2058.5 -45) (end -2058.425 -45.075) (width 0.25) (layer "F.Cu") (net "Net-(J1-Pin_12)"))
 (segment (start -2065.585 -51.866701) (end -2065.325 -51.606701) (width 0.25) (layer "F.Cu") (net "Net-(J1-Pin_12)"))
 (segment (start -2066.5 -53.66) (end -2065.585 -52.745) (width 0.25) (layer "F.Cu") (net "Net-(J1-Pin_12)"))
 (segment (start -2065.701701 -38.5) (end -2060.5 -38.5) (width 0.25) (layer "F.Cu") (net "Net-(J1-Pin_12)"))
 (segment (start -2065.325 -51.606701) (end -2065.325 -50) (width 0.25) (layer "F.Cu") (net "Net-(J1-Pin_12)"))
 (segment (start -2060.5 -38.5) (end -2059 -40) (width 0.25) (layer "F.Cu") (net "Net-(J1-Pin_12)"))
 (segment (start -2067.038604 -49.945) (end -2068.46 -48.523604) (width 0.25) (layer "F.Cu") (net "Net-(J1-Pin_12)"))
 (segment (start -2056.5 -44.7125) (end -2056.8625 -45.075) (width 0.5) (layer "F.Cu") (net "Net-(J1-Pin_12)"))
 (segment (start -2066.5 -46.04) (end -2067.5 -46.04) (width 0.2) (layer "F.Cu") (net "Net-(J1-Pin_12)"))
 (segment (start -2065.38 -49.945) (end -2067.038604 -49.945) (width 0.25) (layer "F.Cu") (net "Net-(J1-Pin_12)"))
 (segment (start -2058.425 -45.075) (end -2056.8625 -45.075) (width 0.25) (layer "F.Cu") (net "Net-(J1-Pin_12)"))
 (segment (start -2067.5 -46.04) (end -2068.46 -46.04) (width 0.2) (layer "F.Cu") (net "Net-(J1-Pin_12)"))
 (segment (start -2069 -45.5) (end -2069 -41.798299) (width 0.25) (layer "F.Cu") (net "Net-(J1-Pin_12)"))
 (segment (start -2065.325 -50) (end -2065.38 -49.945) (width 0.25) (layer "F.Cu") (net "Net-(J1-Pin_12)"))
 (segment (start -2065.585 -52.745) (end -2065.585 -51.866701) (width 0.25) (layer "F.Cu") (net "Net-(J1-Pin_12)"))
 (segment (start -2056.125001 -47.675) (end -2056.8625 -47.675) (width 0.25) (layer "F.Cu") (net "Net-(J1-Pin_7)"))
 (segment (start -2062.92 -48.58) (end -2059.5 -52) (width 0.25) (layer "F.Cu") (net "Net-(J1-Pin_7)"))
 (segment (start -2054.7 -52) (end -2054.7 -49.1) (width 0.25) (layer "F.Cu") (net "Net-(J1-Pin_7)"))
 (segment (start -2054.7 -49.1) (end -2056.125001 -47.675) (width 0.25) (layer "F.Cu") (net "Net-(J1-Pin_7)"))
 (segment (start -2059.5 -52) (end -2054.7 -52) (width 0.25) (layer "F.Cu") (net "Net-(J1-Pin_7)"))
 (segment (start -2063.96 -48.58) (end -2062.92 -48.58) (width 0.25) (layer "F.Cu") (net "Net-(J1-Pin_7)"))
 (segment (start -2064.555 -49.945) (end -2062.555 -49.945) (width 0.25) (layer "F.Cu") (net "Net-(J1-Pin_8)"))
 (segment (start -2054 -48.5) (end -2055.475 -47.025) (width 0.25) (layer "F.Cu") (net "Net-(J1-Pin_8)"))
 (segment (start -2062.555 -49.945) (end -2062.5 -50) (width 0.25) (layer "F.Cu") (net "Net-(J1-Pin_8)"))
 (segment (start -2066.5 -48.58) (end -2065.92 -48.58) (width 0.25) (layer "F.Cu") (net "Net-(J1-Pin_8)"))
 (segment (start -2055.475 -47.025) (end -2056.8625 -47.025) (width 0.25) (layer "F.Cu") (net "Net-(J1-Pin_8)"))
 (segment (start -2054 -52.136396) (end -2054 -48.5) (width 0.25) (layer "F.Cu") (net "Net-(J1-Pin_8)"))
 (segment (start -2054.313604 -52.45) (end -2054 -52.136396) (width 0.25) (layer "F.Cu") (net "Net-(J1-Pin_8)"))
 (segment (start -2059.736828 -52.45) (end -2054.313604 -52.45) (width 0.25) (layer "F.Cu") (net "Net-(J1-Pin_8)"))
 (segment (start -2062.5 -50) (end -2062.186828 -50) (width 0.25) (layer "F.Cu") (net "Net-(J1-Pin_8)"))
 (segment (start -2065.92 -48.58) (end -2064.555 -49.945) (width 0.25) (layer "F.Cu") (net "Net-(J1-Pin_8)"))
 (segment (start -2062.186828 -50) (end -2059.736828 -52.45) (width 0.25) (layer "F.Cu") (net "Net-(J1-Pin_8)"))
 (segment (start -2065.135 -52.295) (end -2065.135 -56.865) (width 0.25) (layer "F.Cu") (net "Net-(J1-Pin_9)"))
 (segment (start -2054.95 -37.55) (end -2054.95 -46) (width 0.25) (layer "F.Cu") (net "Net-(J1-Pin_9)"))
 (segment (start -2055 -36.5) (end -2055.5 -37) (width 0.25) (layer "F.Cu") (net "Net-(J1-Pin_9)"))
 (segment (start -2041.5 -37.5) (end -2042.5 -36.5) (width 0.25) (layer "F.Cu") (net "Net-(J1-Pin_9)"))
 (segment (start -2041.5 -60.5) (end -2041.5 -37.5) (width 0.25) (layer "F.Cu") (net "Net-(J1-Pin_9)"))
 (segment (start -2054.95 -46) (end -2055.5 -46) (width 0.25) (layer "F.Cu") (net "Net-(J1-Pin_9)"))
 (segment (start -2059.625 -62.375) (end -2043.375 -62.375) (width 0.25) (layer "F.Cu") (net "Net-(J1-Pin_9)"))
 (segment (start -2065.135 -56.865) (end -2059.625 -62.375) (width 0.25) (layer "F.Cu") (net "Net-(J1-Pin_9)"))
 (segment (start -2042.5 -36.5) (end -2055 -36.5) (width 0.25) (layer "F.Cu") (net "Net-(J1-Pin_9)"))
 (segment (start -2055.5 -46) (end -2055.875 -46.375) (width 0.25) (layer "F.Cu") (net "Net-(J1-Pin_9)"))
 (segment (start -2063.96 -51.12) (end -2065.135 -52.295) (width 0.25) (layer "F.Cu") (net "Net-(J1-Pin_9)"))
 (segment (start -2043.375 -62.375) (end -2041.5 -60.5) (width 0.25) (layer "F.Cu") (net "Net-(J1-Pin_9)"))
 (segment (start -2055.875 -46.375) (end -2056.8625 -46.375) (width 0.25) (layer "F.Cu") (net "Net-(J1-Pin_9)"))
 (segment (start -2055.5 -37) (end -2054.95 -37.55) (width 0.25) (layer "F.Cu") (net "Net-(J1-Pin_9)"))
 (segment (start -2066 -37.5) (end -2060.5 -37.5) (width 0.25) (layer "F.Cu") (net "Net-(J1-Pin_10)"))
 (segment (start -2070 -41.5) (end -2066 -37.5) (width 0.25) (layer "F.Cu") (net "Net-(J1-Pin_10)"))
 (segment (start -2056.171188 -45.725) (end -2056.8625 -45.725) (width 0.25) (layer "F.Cu") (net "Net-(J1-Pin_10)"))
 (segment (start -2057.6375 -44.1375) (end -2056.261828 -44.1375) (width 0.25) (layer "F.Cu") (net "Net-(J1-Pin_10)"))
 (segment (start -2066.5 -51.12) (end -2070 -47.62) (width 0.25) (layer "F.Cu") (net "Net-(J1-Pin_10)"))
 (segment (start -2055.5 -45.053812) (end -2056.171188 -45.725) (width 0.25) (layer "F.Cu") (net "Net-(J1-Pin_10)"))
 (segment (start -2058 -44.5) (end -2057.6375 -44.1375) (width 0.25) (layer "F.Cu") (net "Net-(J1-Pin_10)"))
 (segment (start -2058 -40) (end -2058 -44.5) (width 0.25) (layer "F.Cu") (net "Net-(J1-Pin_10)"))
 (segment (start -2056.261828 -44.1375) (end -2055.5 -44.899328) (width 0.25) (layer "F.Cu") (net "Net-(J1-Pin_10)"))
 (segment (start -2070 -47.62) (end -2070 -41.5) (width 0.25) (layer "F.Cu") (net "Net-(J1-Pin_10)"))
 (segment (start -2055.5 -44.899328) (end -2055.5 -45.053812) (width 0.25) (layer "F.Cu") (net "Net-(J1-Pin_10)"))
 (segment (start -2060.5 -37.5) (end -2058 -40) (width 0.25) (layer "F.Cu") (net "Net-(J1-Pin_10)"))
 (segment (start -2050.075 -45.399999) (end -2050.400001 -45.725) (width 0.25) (layer "F.Cu") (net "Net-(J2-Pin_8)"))
 (segment (start -2050.075 -43.955) (end -2050.075 -45.399999) (width 0.25) (layer "F.Cu") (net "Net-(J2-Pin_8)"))
 (segment (start -2050.400001 -45.725) (end -2051.1375 -45.725) (width 0.25) (layer "F.Cu") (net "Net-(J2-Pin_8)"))
 (segment (start -2046 -39.88) (end -2050.075 -43.955) (width 0.25) (layer "F.Cu") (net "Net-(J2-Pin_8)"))
 (segment (start -2049.955 -46.375) (end -2051.1375 -46.375) (width 0.25) (layer "F.Cu") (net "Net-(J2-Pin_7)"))
 (segment (start -2046 -42.42) (end -2049.955 -46.375) (width 0.25) (layer "F.Cu") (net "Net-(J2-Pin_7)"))
 (segment (start -2048.065 -47.025) (end -2051.1375 -47.025) (width 0.25) (layer "F.Cu") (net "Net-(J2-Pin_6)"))
 (segment (start -2046 -44.96) (end -2048.065 -47.025) (width 0.25) (layer "F.Cu") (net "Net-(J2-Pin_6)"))
 (segment (start -2046 -47.5) (end -2046.175 -47.675) (width 0.25) (layer "F.Cu") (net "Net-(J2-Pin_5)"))
 (segment (start -2046.175 -47.675) (end -2051.1375 -47.675) (width 0.25) (layer "F.Cu") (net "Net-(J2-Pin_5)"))
 (segment (start -2046 -50.04) (end -2048.46 -50.04) (width 0.25) (layer "F.Cu") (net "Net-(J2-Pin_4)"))
 (segment (start -2048.46 -50.04) (end -2049 -49.5) (width 0.25) (layer "F.Cu") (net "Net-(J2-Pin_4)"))
 (segment (start -2049 -48.863604) (end -2049.538604 -48.325) (width 0.25) (layer "F.Cu") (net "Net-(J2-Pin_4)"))
 (segment (start -2049 -49.5) (end -2049 -48.863604) (width 0.25) (layer "F.Cu") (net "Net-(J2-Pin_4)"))
 (segment (start -2049.538604 -48.325) (end -2051.1375 -48.325) (width 0.25) (layer "F.Cu") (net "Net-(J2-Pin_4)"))
 (segment (start -2049.5 -49) (end -2049.525 -48.975) (width 0.25) (layer "F.Cu") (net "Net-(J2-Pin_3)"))
 (segment (start -2046 -52.58) (end -2049.42 -52.58) (width 0.25) (layer "F.Cu") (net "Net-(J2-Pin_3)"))
 (segment (start -2049.42 -52.58) (end -2049.5 -52.5) (width 0.25) (layer "F.Cu") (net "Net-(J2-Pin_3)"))
 (segment (start -2049.525 -48.975) (end -2051.1375 -48.975) (width 0.25) (layer "F.Cu") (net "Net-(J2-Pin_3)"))
 (segment (start -2049.5 -52.5) (end -2049.5 -49) (width 0.25) (layer "F.Cu") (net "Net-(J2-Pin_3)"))
 (segment (start -2050 -50.025001) (end -2050.400001 -49.625) (width 0.25) (layer "F.Cu") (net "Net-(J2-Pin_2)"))
 (segment (start -2050.400001 -49.625) (end -2051.1375 -49.625) (width 0.25) (layer "F.Cu") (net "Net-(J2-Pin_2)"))
 (segment (start -2046 -55.12) (end -2049.88 -55.12) (width 0.25) (layer "F.Cu") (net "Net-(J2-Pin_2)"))
 (segment (start -2049.88 -55.12) (end -2050 -55) (width 0.25) (layer "F.Cu") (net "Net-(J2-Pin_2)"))
 (segment (start -2050 -55) (end -2050 -50.025001) (width 0.25) (layer "F.Cu") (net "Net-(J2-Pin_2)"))
 (segment (start -2048.84 -57.66) (end -2051.1375 -55.3625) (width 0.25) (layer "F.Cu") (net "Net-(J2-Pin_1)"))
 (segment (start -2051.1375 -55.3625) (end -2051.1375 -50.925) (width 0.25) (layer "F.Cu") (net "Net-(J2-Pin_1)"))
 (segment (start -2046 -57.66) (end -2048.84 -57.66) (width 0.25) (layer "F.Cu") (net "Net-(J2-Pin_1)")))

